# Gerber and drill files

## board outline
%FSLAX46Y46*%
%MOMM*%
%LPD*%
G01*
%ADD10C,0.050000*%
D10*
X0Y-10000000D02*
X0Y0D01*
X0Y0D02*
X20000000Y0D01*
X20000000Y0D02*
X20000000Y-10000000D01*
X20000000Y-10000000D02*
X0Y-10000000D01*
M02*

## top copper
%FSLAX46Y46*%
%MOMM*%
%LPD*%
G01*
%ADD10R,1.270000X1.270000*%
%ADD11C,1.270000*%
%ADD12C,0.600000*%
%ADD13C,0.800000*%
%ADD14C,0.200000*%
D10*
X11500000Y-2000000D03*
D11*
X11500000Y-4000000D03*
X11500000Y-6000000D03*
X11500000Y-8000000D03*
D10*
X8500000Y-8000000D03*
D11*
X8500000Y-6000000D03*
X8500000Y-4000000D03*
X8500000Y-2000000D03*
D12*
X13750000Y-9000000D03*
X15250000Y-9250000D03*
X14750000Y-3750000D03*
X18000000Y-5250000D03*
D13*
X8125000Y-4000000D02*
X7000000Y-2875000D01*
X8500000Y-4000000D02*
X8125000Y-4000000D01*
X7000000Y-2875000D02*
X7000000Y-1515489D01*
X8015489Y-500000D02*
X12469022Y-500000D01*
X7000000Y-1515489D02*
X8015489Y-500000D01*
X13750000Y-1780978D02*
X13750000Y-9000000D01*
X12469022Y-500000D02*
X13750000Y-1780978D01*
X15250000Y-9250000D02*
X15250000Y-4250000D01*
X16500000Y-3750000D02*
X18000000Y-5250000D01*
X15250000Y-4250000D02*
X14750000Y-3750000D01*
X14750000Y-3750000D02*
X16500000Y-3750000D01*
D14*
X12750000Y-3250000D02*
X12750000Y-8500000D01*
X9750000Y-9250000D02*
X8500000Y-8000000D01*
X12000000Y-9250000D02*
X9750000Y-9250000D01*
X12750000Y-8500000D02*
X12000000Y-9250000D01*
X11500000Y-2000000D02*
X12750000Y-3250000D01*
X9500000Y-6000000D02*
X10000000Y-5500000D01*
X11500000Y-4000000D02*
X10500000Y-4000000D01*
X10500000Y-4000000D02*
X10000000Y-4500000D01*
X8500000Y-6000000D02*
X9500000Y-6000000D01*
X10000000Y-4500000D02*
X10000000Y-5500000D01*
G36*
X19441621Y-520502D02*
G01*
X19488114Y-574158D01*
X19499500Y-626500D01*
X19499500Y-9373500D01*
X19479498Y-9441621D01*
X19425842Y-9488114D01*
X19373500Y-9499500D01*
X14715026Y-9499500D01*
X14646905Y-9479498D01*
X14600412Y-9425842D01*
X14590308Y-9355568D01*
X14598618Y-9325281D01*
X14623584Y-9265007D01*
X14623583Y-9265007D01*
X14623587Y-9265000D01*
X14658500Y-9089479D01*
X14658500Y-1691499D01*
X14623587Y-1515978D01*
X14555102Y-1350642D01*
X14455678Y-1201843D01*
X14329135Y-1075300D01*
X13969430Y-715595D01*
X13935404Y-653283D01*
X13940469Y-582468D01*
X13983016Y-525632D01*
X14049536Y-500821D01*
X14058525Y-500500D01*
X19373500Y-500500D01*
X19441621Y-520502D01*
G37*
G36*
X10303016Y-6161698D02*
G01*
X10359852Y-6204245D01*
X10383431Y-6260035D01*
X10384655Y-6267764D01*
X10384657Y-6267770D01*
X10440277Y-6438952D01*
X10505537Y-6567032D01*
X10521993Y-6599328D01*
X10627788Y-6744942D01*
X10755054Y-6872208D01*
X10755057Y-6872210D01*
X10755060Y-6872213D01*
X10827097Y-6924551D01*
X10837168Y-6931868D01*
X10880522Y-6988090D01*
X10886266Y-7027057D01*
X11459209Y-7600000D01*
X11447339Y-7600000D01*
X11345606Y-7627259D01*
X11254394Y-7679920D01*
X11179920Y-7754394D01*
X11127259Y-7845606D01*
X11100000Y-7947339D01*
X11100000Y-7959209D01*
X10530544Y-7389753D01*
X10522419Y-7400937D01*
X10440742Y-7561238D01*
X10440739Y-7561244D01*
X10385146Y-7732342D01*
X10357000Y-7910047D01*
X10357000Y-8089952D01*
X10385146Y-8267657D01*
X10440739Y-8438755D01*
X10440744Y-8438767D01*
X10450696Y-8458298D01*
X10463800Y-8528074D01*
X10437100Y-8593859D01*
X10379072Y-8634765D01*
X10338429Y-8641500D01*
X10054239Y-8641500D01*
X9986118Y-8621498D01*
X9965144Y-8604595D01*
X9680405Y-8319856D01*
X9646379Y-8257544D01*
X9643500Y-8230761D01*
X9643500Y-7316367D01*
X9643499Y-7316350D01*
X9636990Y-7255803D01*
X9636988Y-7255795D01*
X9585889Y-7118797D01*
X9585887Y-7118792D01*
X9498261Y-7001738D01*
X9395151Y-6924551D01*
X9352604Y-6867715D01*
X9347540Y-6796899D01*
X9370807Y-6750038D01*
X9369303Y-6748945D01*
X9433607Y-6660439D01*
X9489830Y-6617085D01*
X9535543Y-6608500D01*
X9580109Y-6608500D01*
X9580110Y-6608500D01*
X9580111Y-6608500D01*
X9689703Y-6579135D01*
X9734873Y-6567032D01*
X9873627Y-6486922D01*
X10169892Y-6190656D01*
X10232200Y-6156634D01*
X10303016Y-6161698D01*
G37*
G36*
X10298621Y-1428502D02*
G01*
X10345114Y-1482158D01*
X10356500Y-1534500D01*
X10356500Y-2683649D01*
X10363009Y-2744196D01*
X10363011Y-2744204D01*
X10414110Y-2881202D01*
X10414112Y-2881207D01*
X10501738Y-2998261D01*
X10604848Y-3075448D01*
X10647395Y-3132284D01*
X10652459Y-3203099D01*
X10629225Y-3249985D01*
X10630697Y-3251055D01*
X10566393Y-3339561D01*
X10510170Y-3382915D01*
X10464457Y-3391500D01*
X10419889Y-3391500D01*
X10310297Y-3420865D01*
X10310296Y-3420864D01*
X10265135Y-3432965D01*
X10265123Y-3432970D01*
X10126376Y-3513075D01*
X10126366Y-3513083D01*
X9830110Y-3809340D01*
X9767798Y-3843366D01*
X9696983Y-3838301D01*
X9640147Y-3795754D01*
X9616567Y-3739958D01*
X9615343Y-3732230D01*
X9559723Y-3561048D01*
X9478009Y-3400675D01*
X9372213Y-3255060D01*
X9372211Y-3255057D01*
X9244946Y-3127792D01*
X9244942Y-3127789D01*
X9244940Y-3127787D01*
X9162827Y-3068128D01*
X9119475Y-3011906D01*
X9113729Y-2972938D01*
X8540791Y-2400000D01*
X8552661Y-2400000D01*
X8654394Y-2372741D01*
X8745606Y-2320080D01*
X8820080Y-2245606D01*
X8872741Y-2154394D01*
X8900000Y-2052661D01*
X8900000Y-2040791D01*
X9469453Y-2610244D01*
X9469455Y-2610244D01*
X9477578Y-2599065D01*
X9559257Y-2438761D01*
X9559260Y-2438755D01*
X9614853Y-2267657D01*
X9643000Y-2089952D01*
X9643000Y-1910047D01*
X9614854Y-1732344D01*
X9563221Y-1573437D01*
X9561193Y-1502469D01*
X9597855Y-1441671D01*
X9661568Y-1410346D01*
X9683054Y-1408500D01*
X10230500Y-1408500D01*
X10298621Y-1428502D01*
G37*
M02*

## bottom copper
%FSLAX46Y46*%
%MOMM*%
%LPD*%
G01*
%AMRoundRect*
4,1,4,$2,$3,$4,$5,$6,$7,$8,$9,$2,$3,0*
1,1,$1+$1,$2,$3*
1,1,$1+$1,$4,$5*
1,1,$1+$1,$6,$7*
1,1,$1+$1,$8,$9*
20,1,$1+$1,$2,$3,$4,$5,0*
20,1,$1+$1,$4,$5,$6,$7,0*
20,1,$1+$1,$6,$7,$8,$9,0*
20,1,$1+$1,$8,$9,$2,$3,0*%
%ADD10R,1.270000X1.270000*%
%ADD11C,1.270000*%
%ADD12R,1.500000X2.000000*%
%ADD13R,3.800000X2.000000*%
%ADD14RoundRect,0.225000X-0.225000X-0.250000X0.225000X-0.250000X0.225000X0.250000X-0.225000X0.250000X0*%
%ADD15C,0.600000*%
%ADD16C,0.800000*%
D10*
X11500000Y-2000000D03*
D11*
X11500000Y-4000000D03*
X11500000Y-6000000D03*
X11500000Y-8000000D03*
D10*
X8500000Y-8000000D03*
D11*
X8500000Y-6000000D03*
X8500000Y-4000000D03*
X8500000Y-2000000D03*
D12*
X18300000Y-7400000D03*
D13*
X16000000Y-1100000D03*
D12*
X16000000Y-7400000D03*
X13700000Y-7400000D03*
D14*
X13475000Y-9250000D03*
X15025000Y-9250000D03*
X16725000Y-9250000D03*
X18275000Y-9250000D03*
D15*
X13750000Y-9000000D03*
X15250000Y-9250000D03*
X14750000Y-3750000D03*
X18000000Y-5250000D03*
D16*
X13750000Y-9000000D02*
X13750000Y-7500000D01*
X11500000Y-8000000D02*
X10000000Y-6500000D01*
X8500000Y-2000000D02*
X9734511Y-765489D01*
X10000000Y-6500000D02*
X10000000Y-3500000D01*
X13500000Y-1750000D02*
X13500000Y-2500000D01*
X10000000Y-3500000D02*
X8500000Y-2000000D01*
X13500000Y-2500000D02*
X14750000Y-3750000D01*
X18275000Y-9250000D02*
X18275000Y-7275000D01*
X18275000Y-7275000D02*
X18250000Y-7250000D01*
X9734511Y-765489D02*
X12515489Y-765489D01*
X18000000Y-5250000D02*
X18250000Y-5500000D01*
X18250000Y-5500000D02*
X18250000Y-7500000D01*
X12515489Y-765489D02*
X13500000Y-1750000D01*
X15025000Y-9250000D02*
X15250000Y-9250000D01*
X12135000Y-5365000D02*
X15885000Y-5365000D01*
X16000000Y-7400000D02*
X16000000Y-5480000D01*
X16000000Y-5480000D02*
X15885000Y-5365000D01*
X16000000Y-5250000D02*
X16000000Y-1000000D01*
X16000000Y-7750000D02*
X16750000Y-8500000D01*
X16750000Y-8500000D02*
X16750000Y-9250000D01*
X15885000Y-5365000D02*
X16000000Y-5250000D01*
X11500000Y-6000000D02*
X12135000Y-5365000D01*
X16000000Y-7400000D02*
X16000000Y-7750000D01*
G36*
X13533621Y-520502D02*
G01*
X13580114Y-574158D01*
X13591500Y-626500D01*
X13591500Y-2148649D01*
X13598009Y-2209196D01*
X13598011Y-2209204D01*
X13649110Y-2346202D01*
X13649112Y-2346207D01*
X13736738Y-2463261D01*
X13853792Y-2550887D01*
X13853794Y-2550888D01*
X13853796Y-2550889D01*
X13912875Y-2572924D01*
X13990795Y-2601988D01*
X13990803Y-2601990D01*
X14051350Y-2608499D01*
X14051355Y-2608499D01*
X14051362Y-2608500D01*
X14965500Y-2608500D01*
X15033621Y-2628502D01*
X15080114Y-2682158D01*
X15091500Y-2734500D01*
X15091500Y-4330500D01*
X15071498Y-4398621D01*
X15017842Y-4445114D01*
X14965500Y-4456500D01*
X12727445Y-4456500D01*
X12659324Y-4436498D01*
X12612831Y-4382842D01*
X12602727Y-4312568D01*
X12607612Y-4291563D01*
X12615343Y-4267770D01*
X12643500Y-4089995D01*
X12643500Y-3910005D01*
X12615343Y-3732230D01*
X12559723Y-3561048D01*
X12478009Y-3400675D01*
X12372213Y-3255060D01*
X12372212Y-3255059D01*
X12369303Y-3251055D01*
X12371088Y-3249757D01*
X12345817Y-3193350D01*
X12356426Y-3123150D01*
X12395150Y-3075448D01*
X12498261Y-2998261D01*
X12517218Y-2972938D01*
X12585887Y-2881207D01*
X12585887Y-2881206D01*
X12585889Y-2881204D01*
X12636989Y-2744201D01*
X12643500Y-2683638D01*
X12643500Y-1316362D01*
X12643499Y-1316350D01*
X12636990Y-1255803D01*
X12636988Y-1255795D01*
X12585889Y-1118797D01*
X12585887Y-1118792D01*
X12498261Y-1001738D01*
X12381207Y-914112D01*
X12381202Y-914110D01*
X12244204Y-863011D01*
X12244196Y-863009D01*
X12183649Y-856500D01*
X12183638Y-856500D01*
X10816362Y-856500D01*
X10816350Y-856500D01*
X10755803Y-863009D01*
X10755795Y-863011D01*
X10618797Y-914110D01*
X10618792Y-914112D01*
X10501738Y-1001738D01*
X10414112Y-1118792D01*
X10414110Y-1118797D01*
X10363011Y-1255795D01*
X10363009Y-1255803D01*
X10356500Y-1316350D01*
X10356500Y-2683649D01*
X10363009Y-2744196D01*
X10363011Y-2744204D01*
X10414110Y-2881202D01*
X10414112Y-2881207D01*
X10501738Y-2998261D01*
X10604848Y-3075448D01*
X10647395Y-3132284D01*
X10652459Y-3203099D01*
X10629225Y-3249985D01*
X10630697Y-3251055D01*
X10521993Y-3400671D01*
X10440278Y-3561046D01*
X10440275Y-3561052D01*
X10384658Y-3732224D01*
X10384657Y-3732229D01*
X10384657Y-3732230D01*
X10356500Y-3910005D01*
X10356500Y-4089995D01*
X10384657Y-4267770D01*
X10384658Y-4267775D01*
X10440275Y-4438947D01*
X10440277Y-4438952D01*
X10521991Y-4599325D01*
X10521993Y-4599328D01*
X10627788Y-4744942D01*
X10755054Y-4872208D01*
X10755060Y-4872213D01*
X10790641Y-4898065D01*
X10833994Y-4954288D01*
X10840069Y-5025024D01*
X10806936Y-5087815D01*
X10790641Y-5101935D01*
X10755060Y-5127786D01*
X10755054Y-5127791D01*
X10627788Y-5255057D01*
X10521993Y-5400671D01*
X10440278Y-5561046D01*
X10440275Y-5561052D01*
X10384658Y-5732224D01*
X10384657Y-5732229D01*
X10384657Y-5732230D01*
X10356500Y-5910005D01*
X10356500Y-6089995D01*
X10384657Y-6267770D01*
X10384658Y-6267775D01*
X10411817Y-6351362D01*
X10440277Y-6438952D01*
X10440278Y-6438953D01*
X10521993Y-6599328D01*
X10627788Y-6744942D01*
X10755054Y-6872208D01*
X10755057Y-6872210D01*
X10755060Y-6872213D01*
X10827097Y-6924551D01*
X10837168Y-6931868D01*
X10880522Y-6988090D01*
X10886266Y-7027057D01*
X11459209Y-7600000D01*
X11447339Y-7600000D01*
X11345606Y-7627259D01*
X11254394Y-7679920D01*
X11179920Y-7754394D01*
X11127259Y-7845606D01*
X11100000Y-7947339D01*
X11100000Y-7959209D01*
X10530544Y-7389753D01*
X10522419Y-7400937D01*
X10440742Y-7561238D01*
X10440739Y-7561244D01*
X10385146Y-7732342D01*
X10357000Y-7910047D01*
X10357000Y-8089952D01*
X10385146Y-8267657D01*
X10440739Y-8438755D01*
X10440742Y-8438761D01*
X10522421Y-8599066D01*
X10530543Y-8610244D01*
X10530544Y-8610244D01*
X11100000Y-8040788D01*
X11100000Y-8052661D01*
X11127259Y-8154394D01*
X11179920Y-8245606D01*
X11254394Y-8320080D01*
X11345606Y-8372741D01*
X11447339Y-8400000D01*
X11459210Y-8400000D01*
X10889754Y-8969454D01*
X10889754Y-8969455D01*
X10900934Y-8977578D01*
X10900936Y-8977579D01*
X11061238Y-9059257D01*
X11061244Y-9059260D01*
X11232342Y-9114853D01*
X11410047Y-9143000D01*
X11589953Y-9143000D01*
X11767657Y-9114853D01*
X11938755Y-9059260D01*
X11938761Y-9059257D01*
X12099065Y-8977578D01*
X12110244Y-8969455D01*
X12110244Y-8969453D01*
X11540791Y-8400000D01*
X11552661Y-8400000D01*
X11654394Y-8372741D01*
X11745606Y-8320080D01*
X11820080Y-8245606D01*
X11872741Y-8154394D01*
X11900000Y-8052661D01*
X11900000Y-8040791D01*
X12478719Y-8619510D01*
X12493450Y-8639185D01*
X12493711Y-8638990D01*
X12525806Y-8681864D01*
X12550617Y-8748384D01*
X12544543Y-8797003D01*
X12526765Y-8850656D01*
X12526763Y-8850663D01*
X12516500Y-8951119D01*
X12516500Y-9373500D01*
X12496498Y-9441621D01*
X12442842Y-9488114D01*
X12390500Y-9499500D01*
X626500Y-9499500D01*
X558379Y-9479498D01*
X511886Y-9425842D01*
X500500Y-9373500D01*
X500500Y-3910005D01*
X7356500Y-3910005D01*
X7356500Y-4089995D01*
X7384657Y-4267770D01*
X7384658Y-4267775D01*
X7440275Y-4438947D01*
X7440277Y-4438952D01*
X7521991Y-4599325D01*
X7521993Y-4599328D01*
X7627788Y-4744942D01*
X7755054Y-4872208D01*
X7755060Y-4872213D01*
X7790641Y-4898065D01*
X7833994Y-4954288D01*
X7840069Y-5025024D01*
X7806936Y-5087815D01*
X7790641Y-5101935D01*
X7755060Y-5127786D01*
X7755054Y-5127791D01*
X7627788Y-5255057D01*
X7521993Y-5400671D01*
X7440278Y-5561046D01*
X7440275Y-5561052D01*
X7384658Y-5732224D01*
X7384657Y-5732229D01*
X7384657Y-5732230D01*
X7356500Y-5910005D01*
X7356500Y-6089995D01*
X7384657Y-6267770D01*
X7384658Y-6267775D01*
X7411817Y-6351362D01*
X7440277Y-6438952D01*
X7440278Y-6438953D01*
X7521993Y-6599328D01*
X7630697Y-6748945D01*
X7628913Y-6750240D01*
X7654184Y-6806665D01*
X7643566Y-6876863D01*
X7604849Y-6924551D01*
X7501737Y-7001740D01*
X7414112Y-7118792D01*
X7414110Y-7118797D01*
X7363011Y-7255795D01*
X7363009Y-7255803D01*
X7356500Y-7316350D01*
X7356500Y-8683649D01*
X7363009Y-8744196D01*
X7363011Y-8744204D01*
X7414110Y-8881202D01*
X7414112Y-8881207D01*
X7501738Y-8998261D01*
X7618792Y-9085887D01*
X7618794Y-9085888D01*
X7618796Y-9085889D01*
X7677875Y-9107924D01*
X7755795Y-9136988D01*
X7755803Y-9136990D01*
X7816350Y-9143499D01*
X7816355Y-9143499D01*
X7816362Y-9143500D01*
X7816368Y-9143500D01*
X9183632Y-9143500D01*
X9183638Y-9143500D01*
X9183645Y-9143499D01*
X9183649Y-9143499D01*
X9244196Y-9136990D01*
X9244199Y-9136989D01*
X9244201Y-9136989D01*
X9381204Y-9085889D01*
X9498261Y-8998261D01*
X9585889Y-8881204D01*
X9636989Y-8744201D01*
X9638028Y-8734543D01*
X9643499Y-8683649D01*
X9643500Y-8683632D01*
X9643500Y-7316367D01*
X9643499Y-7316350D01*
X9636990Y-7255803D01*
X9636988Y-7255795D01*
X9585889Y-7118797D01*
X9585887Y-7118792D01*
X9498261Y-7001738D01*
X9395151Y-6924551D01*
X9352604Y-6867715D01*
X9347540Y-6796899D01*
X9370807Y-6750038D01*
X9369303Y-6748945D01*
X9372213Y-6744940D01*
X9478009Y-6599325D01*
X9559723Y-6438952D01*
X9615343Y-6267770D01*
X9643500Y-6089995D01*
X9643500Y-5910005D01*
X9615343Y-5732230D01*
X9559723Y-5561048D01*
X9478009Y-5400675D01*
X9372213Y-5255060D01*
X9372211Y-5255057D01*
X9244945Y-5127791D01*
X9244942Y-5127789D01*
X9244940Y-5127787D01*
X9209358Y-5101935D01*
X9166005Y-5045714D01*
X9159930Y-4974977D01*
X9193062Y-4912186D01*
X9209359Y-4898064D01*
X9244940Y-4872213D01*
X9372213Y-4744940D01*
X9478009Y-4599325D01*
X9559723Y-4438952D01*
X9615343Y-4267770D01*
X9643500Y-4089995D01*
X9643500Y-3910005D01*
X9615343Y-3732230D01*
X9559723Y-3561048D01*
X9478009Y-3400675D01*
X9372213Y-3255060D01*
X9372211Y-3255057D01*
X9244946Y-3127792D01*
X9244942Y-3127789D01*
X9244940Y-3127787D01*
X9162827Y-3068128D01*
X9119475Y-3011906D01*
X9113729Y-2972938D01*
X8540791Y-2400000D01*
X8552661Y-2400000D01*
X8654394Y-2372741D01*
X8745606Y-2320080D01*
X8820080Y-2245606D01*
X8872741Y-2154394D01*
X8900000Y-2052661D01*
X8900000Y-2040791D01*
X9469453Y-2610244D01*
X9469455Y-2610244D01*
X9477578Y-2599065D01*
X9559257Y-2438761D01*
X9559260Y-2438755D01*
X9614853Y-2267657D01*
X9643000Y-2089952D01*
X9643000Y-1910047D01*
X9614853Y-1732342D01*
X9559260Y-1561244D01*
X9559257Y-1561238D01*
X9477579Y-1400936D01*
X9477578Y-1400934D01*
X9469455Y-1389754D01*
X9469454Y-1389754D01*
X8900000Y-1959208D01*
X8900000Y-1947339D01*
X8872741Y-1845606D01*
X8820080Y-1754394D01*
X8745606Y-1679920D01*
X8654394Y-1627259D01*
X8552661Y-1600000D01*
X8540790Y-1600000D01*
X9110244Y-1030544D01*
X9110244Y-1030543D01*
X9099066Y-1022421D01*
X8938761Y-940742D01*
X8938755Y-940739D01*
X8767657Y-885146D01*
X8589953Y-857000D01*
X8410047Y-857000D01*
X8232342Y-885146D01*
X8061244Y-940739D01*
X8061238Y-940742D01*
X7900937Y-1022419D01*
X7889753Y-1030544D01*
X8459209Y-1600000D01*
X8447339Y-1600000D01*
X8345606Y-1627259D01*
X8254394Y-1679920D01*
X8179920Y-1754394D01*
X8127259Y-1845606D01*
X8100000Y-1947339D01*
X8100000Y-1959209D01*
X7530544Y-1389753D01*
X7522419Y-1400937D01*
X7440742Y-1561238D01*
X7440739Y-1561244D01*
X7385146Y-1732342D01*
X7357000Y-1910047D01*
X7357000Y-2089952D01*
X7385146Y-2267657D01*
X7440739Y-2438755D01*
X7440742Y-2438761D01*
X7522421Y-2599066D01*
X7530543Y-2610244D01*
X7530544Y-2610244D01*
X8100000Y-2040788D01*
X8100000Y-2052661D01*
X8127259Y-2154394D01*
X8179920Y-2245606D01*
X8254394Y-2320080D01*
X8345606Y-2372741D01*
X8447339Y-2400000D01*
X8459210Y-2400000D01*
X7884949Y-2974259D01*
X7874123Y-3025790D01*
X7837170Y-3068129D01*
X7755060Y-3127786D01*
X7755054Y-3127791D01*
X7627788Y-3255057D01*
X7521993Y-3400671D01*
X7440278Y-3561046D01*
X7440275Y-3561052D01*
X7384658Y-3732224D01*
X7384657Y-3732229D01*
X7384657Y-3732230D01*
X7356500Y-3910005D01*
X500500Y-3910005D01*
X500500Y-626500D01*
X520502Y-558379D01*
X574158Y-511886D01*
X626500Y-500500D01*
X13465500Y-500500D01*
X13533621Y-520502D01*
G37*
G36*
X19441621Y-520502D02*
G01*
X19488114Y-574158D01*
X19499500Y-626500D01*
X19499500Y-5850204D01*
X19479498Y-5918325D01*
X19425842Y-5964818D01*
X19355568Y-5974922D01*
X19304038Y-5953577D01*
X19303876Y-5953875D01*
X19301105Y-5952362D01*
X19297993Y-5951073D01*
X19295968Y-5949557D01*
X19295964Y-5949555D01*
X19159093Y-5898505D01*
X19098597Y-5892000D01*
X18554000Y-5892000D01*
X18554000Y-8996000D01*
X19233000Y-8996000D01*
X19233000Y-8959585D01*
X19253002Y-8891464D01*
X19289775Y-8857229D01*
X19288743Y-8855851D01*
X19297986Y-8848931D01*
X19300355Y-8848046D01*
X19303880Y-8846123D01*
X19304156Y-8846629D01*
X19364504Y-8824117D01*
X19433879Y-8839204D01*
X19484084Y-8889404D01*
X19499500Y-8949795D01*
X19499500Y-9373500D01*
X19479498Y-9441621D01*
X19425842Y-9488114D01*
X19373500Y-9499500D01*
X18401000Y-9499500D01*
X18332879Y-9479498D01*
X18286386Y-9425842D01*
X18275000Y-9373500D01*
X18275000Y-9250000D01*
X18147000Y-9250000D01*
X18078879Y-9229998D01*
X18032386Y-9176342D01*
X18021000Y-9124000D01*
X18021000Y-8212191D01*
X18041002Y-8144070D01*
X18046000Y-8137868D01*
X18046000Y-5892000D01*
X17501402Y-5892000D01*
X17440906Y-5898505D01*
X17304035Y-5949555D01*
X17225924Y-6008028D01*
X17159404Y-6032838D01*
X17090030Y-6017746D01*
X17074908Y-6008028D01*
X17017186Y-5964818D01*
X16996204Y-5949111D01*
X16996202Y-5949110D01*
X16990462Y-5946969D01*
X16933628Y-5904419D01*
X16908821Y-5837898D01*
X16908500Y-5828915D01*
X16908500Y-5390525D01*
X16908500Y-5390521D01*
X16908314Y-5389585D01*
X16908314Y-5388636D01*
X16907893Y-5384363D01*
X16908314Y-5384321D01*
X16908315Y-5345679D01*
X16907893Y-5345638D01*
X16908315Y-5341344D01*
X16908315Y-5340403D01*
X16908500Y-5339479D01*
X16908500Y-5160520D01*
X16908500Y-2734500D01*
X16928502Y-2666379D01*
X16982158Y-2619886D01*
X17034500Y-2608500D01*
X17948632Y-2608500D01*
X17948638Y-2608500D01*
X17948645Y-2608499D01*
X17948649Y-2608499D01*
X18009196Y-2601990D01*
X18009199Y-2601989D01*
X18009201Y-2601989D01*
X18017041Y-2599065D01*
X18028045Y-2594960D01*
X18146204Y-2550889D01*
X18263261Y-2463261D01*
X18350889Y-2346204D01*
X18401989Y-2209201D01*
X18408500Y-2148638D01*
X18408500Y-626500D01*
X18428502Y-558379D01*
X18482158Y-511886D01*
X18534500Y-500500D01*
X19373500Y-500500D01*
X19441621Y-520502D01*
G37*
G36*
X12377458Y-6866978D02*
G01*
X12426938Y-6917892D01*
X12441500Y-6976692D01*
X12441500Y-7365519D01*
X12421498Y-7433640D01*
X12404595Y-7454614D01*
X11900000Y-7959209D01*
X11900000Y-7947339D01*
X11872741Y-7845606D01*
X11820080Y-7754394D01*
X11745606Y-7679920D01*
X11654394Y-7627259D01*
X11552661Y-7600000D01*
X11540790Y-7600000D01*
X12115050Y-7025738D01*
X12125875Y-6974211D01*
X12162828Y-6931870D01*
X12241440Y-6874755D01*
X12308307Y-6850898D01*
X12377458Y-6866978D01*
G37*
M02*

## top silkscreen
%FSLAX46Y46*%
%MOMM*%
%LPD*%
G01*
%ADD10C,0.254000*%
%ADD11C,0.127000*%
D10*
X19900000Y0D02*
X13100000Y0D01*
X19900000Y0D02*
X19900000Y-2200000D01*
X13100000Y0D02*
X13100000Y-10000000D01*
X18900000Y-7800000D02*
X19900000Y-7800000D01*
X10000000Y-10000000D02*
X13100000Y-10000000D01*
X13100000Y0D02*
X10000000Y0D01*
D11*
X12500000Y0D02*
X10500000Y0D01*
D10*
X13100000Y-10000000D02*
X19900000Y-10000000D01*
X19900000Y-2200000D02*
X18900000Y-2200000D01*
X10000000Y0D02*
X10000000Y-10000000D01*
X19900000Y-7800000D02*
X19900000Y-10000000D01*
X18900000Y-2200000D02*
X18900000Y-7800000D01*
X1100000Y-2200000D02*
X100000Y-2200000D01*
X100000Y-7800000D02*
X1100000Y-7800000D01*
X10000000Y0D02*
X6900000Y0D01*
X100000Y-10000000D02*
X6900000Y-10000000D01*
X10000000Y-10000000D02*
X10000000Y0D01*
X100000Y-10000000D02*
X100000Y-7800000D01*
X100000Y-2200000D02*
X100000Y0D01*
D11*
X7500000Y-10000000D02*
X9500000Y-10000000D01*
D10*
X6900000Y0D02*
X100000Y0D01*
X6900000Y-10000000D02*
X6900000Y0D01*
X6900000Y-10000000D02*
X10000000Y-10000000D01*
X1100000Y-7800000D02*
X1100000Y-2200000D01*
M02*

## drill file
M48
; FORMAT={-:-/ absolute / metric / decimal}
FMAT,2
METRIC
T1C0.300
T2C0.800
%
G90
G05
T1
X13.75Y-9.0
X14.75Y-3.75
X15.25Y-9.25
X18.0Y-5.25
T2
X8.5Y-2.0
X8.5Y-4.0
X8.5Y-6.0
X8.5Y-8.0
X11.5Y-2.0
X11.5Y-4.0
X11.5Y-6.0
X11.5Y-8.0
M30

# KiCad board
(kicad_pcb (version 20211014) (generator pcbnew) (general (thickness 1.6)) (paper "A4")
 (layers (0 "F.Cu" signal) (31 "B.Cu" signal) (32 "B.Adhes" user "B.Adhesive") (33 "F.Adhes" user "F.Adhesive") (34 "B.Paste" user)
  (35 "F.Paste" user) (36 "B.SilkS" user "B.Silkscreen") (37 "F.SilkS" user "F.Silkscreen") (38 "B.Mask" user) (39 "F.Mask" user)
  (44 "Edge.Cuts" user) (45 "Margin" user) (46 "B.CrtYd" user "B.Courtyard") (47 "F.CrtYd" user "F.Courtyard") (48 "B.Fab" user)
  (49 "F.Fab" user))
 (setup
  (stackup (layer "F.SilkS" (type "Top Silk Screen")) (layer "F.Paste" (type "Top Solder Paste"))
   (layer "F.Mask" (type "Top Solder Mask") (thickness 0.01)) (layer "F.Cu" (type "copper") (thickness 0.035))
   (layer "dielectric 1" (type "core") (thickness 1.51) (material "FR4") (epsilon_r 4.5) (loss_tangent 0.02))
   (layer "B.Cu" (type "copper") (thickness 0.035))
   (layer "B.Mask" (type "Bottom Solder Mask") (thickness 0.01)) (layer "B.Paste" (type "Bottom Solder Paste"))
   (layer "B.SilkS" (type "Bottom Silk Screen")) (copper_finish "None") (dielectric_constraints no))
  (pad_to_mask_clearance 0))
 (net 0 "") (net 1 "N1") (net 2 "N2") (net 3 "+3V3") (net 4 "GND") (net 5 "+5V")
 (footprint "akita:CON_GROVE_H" (layer "F.Cu") (at 11.5 5 -90)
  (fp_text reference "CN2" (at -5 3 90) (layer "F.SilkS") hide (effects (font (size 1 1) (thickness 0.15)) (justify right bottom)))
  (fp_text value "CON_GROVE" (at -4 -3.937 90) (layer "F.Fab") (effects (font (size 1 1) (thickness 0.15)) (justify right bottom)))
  (fp_line (start -5 -8.4) (end -5 -1.6) (layer "F.SilkS") (width 0.254))
  (fp_line (start -5 -8.4) (end -2.8 -8.4) (layer "F.SilkS") (width 0.254))
  (fp_line (start -5 -1.6) (end 5 -1.6) (layer "F.SilkS") (width 0.254))
  (fp_line (start 2.8 -7.4) (end 2.8 -8.4) (layer "F.SilkS") (width 0.254))
  (fp_line (start 5 1.5) (end 5 -1.6) (layer "F.SilkS") (width 0.254))
  (fp_line (start -5 -1.6) (end -5 1.5) (layer "F.SilkS") (width 0.254))
  (fp_line (start -5 -1) (end -5 1) (layer "F.SilkS") (width 0.127))
  (fp_line (start 5 -1.6) (end 5 -8.4) (layer "F.SilkS") (width 0.254))
  (fp_line (start -2.8 -8.4) (end -2.8 -7.4) (layer "F.SilkS") (width 0.254))
  (fp_line (start -5 1.5) (end 5 1.5) (layer "F.SilkS") (width 0.254))
  (fp_line (start 2.8 -8.4) (end 5 -8.4) (layer "F.SilkS") (width 0.254))
  (fp_line (start -2.8 -7.4) (end 2.8 -7.4) (layer "F.SilkS") (width 0.254))
  (pad "1" thru_hole rect locked (at -3 0 270) (size 1.27 1.27) (drill 0.8) (layers *.Cu *.Mask) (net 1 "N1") (solder_mask_margin 0.1016))
  (pad "2" thru_hole circle locked (at -1 0 270) (size 1.27 1.27) (drill 0.8) (layers *.Cu *.Mask) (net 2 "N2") (solder_mask_margin 0.1016))
  (pad "3" thru_hole circle locked (at 1 0 270) (size 1.27 1.27) (drill 0.8) (layers *.Cu *.Mask) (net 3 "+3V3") (solder_mask_margin 0.1016))
  (pad "4" thru_hole circle locked (at 3 0 270) (size 1.27 1.27) (drill 0.8) (layers *.Cu *.Mask) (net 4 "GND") (solder_mask_margin 0.1016)))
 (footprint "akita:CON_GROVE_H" (layer "F.Cu") (at 8.5 5 90)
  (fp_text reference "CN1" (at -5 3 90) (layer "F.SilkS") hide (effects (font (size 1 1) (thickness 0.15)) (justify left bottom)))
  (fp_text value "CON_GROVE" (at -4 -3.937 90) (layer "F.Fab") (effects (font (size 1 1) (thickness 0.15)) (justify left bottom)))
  (fp_line (start 2.8 -7.4) (end 2.8 -8.4) (layer "F.SilkS") (width 0.254))
  (fp_line (start -2.8 -8.4) (end -2.8 -7.4) (layer "F.SilkS") (width 0.254))
  (fp_line (start 5 1.5) (end 5 -1.6) (layer "F.SilkS") (width 0.254))
  (fp_line (start -5 -8.4) (end -5 -1.6) (layer "F.SilkS") (width 0.254))
  (fp_line (start -5 1.5) (end 5 1.5) (layer "F.SilkS") (width 0.254))
  (fp_line (start -5 -8.4) (end -2.8 -8.4) (layer "F.SilkS") (width 0.254))
  (fp_line (start 2.8 -8.4) (end 5 -8.4) (layer "F.SilkS") (width 0.254))
  (fp_line (start -5 -1) (end -5 1) (layer "F.SilkS") (width 0.127))
  (fp_line (start 5 -1.6) (end 5 -8.4) (layer "F.SilkS") (width 0.254))
  (fp_line (start -5 -1.6) (end 5 -1.6) (layer "F.SilkS") (width 0.254))
  (fp_line (start -5 -1.6) (end -5 1.5) (layer "F.SilkS") (width 0.254))
  (fp_line (start -2.8 -7.4) (end 2.8 -7.4) (layer "F.SilkS") (width 0.254))
  (pad "1" thru_hole rect locked (at -3 0 90) (size 1.27 1.27) (drill 0.8) (layers *.Cu *.Mask) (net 1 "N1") (solder_mask_margin 0.1016))
  (pad "2" thru_hole circle locked (at -1 0 90) (size 1.27 1.27) (drill 0.8) (layers *.Cu *.Mask) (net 2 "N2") (solder_mask_margin 0.1016))
  (pad "3" thru_hole circle locked (at 1 0 90) (size 1.27 1.27) (drill 0.8) (layers *.Cu *.Mask) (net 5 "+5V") (solder_mask_margin 0.1016))
  (pad "4" thru_hole circle locked (at 3 0 90) (size 1.27 1.27) (drill 0.8) (layers *.Cu *.Mask) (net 4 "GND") (solder_mask_margin 0.1016)))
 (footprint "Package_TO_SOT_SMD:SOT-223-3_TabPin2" (layer "B.Cu") (at 16 4.25 90)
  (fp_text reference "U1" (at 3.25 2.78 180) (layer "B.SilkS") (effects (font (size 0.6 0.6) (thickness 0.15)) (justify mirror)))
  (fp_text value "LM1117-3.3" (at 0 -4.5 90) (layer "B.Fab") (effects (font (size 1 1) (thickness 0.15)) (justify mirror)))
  (pad "1" smd rect locked (at -3.15 2.3 90) (size 2 1.5) (layers "B.Cu" "B.Paste" "B.Mask") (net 4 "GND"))
  (pad "2" smd rect locked (at 3.15 0 90) (size 2 3.8) (layers "B.Cu" "B.Paste" "B.Mask") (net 3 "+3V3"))
  (pad "2" smd rect locked (at -3.15 0 90) (size 2 1.5) (layers "B.Cu" "B.Paste" "B.Mask") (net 3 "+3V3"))
  (pad "3" smd rect locked (at -3.15 -2.3 90) (size 2 1.5) (layers "B.Cu" "B.Paste" "B.Mask") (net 5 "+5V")))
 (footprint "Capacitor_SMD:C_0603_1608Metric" (layer "B.Cu") (at 14.25 9.25)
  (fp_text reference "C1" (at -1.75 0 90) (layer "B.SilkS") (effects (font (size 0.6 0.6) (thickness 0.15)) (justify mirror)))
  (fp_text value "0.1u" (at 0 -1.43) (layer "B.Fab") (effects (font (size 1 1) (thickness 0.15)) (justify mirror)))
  (pad "1" smd roundrect locked (at -0.775 0) (size 0.9 0.95) (layers "B.Cu" "B.Paste" "B.Mask") (roundrect_rratio 0.25) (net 5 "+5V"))
  (pad "2" smd roundrect locked (at 0.775 0) (size 0.9 0.95) (layers "B.Cu" "B.Paste" "B.Mask") (roundrect_rratio 0.25) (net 4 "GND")))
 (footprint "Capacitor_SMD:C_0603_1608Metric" (layer "B.Cu") (at 17.5 9.25)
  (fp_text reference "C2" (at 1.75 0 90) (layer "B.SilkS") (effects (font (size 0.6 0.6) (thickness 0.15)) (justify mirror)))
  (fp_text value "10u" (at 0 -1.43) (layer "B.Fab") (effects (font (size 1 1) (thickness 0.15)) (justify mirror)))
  (pad "1" smd roundrect locked (at -0.775 0) (size 0.9 0.95) (layers "B.Cu" "B.Paste" "B.Mask") (roundrect_rratio 0.25) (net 3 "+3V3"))
  (pad "2" smd roundrect locked (at 0.775 0) (size 0.9 0.95) (layers "B.Cu" "B.Paste" "B.Mask") (roundrect_rratio 0.25) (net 4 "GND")))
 (gr_line (start 0 10) (end 0 0) (layer "Edge.Cuts") (width 0.05))
 (gr_line (start 0 0) (end 20 0) (layer "Edge.Cuts") (width 0.05))
 (gr_line (start 20 0) (end 20 10) (layer "Edge.Cuts") (width 0.05))
 (gr_line (start 20 10) (end 0 10) (layer "Edge.Cuts") (width 0.05))
 (segment (start 8.125 4) (end 7 2.875) (width 0.8) (layer "F.Cu") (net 5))
 (segment (start 8.5 4) (end 8.125 4) (width 0.8) (layer "F.Cu") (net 5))
 (segment (start 7 2.875) (end 7 1.515489) (width 0.8) (layer "F.Cu") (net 5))
 (segment (start 8.015489 0.5) (end 12.469022 0.5) (width 0.8) (layer "F.Cu") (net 5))
 (segment (start 7 1.515489) (end 8.015489 0.5) (width 0.8) (layer "F.Cu") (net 5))
 (segment (start 13.75 1.780978) (end 13.75 9) (width 0.8) (layer "F.Cu") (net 5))
 (segment (start 12.469022 0.5) (end 13.75 1.780978) (width 0.8) (layer "F.Cu") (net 5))
 (via (at 13.75 9) (size 0.6) (drill 0.3) (layers "F.Cu" "B.Cu") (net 5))
 (segment (start 13.75 9) (end 13.75 7.5) (width 0.8) (layer "B.Cu") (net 5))
 (segment (start 15.25 9.25) (end 15.25 4.25) (width 0.8) (layer "F.Cu") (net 4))
 (segment (start 16.5 3.75) (end 18 5.25) (width 0.8) (layer "F.Cu") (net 4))
 (segment (start 15.25 4.25) (end 14.75 3.75) (width 0.8) (layer "F.Cu") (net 4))
 (segment (start 14.75 3.75) (end 16.5 3.75) (width 0.8) (layer "F.Cu") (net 4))
 (via (at 15.25 9.25) (size 0.6) (drill 0.3) (layers "F.Cu" "B.Cu") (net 4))
 (via (at 14.75 3.75) (size 0.6) (drill 0.3) (layers "F.Cu" "B.Cu") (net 4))
 (via (at 18 5.25) (size 0.6) (drill 0.3) (layers "F.Cu" "B.Cu") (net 4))
 (segment (start 11.5 8) (end 10 6.5) (width 0.8) (layer "B.Cu") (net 4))
 (segment (start 8.5 2) (end 9.734511 0.765489) (width 0.8) (layer "B.Cu") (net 4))
 (segment (start 10 6.5) (end 10 3.5) (width 0.8) (layer "B.Cu") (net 4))
 (segment (start 13.5 1.75) (end 13.5 2.5) (width 0.8) (layer "B.Cu") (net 4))
 (segment (start 10 3.5) (end 8.5 2) (width 0.8) (layer "B.Cu") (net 4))
 (segment (start 13.5 2.5) (end 14.75 3.75) (width 0.8) (layer "B.Cu") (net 4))
 (segment (start 18.275 9.25) (end 18.275 7.275) (width 0.8) (layer "B.Cu") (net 4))
 (segment (start 18.275 7.275) (end 18.25 7.25) (width 0.8) (layer "B.Cu") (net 4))
 (segment (start 9.734511 0.765489) (end 12.515489 0.765489) (width 0.8) (layer "B.Cu") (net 4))
 (segment (start 18 5.25) (end 18.25 5.5) (width 0.8) (layer "B.Cu") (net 4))
 (segment (start 18.25 5.5) (end 18.25 7.5) (width 0.8) (layer "B.Cu") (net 4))
 (segment (start 12.515489 0.765489) (end 13.5 1.75) (width 0.8) (layer "B.Cu") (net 4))
 (segment (start 15.025 9.25) (end 15.25 9.25) (width 0.8) (layer "B.Cu") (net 4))
 (segment (start 12.135 5.365) (end 15.885 5.365) (width 0.8) (layer "B.Cu") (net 3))
 (segment (start 16 7.4) (end 16 5.48) (width 0.8) (layer "B.Cu") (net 3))
 (segment (start 16 5.48) (end 15.885 5.365) (width 0.8) (layer "B.Cu") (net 3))
 (segment (start 16 5.25) (end 16 1) (width 0.8) (layer "B.Cu") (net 3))
 (segment (start 16 7.75) (end 16.75 8.5) (width 0.8) (layer "B.Cu") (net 3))
 (segment (start 16.75 8.5) (end 16.75 9.25) (width 0.8) (layer "B.Cu") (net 3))
 (segment (start 15.885 5.365) (end 16 5.25) (width 0.8) (layer "B.Cu") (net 3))
 (segment (start 11.5 6) (end 12.135 5.365) (width 0.8) (layer "B.Cu") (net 3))
 (segment (start 16 7.4) (end 16 7.75) (width 0.8) (layer "B.Cu") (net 3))
 (segment (start 12.75 3.25) (end 12.75 8.5) (width 0.2) (layer "F.Cu") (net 1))
 (segment (start 9.75 9.25) (end 8.5 8) (width 0.2) (layer "F.Cu") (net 1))
 (segment (start 12 9.25) (end 9.75 9.25) (width 0.2) (layer "F.Cu") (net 1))
 (segment (start 12.75 8.5) (end 12 9.25) (width 0.2) (layer "F.Cu") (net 1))
 (segment (start 11.5 2) (end 12.75 3.25) (width 0.2) (layer "F.Cu") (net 1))
 (segment (start 9.5 6) (end 10 5.5) (width 0.2) (layer "F.Cu") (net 2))
 (segment (start 11.5 4) (end 10.5 4) (width 0.2) (layer "F.Cu") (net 2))
 (segment (start 10.5 4) (end 10 4.5) (width 0.2) (layer "F.Cu") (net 2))
 (segment (start 8.5 6) (end 9.5 6) (width 0.2) (layer "F.Cu") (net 2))
 (segment (start 10 4.5) (end 10 5.5) (width 0.2) (layer "F.Cu") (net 2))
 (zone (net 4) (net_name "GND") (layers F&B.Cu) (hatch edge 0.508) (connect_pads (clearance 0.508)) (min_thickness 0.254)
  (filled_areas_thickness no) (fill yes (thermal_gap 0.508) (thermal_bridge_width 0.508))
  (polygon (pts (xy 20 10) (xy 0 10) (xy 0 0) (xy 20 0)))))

